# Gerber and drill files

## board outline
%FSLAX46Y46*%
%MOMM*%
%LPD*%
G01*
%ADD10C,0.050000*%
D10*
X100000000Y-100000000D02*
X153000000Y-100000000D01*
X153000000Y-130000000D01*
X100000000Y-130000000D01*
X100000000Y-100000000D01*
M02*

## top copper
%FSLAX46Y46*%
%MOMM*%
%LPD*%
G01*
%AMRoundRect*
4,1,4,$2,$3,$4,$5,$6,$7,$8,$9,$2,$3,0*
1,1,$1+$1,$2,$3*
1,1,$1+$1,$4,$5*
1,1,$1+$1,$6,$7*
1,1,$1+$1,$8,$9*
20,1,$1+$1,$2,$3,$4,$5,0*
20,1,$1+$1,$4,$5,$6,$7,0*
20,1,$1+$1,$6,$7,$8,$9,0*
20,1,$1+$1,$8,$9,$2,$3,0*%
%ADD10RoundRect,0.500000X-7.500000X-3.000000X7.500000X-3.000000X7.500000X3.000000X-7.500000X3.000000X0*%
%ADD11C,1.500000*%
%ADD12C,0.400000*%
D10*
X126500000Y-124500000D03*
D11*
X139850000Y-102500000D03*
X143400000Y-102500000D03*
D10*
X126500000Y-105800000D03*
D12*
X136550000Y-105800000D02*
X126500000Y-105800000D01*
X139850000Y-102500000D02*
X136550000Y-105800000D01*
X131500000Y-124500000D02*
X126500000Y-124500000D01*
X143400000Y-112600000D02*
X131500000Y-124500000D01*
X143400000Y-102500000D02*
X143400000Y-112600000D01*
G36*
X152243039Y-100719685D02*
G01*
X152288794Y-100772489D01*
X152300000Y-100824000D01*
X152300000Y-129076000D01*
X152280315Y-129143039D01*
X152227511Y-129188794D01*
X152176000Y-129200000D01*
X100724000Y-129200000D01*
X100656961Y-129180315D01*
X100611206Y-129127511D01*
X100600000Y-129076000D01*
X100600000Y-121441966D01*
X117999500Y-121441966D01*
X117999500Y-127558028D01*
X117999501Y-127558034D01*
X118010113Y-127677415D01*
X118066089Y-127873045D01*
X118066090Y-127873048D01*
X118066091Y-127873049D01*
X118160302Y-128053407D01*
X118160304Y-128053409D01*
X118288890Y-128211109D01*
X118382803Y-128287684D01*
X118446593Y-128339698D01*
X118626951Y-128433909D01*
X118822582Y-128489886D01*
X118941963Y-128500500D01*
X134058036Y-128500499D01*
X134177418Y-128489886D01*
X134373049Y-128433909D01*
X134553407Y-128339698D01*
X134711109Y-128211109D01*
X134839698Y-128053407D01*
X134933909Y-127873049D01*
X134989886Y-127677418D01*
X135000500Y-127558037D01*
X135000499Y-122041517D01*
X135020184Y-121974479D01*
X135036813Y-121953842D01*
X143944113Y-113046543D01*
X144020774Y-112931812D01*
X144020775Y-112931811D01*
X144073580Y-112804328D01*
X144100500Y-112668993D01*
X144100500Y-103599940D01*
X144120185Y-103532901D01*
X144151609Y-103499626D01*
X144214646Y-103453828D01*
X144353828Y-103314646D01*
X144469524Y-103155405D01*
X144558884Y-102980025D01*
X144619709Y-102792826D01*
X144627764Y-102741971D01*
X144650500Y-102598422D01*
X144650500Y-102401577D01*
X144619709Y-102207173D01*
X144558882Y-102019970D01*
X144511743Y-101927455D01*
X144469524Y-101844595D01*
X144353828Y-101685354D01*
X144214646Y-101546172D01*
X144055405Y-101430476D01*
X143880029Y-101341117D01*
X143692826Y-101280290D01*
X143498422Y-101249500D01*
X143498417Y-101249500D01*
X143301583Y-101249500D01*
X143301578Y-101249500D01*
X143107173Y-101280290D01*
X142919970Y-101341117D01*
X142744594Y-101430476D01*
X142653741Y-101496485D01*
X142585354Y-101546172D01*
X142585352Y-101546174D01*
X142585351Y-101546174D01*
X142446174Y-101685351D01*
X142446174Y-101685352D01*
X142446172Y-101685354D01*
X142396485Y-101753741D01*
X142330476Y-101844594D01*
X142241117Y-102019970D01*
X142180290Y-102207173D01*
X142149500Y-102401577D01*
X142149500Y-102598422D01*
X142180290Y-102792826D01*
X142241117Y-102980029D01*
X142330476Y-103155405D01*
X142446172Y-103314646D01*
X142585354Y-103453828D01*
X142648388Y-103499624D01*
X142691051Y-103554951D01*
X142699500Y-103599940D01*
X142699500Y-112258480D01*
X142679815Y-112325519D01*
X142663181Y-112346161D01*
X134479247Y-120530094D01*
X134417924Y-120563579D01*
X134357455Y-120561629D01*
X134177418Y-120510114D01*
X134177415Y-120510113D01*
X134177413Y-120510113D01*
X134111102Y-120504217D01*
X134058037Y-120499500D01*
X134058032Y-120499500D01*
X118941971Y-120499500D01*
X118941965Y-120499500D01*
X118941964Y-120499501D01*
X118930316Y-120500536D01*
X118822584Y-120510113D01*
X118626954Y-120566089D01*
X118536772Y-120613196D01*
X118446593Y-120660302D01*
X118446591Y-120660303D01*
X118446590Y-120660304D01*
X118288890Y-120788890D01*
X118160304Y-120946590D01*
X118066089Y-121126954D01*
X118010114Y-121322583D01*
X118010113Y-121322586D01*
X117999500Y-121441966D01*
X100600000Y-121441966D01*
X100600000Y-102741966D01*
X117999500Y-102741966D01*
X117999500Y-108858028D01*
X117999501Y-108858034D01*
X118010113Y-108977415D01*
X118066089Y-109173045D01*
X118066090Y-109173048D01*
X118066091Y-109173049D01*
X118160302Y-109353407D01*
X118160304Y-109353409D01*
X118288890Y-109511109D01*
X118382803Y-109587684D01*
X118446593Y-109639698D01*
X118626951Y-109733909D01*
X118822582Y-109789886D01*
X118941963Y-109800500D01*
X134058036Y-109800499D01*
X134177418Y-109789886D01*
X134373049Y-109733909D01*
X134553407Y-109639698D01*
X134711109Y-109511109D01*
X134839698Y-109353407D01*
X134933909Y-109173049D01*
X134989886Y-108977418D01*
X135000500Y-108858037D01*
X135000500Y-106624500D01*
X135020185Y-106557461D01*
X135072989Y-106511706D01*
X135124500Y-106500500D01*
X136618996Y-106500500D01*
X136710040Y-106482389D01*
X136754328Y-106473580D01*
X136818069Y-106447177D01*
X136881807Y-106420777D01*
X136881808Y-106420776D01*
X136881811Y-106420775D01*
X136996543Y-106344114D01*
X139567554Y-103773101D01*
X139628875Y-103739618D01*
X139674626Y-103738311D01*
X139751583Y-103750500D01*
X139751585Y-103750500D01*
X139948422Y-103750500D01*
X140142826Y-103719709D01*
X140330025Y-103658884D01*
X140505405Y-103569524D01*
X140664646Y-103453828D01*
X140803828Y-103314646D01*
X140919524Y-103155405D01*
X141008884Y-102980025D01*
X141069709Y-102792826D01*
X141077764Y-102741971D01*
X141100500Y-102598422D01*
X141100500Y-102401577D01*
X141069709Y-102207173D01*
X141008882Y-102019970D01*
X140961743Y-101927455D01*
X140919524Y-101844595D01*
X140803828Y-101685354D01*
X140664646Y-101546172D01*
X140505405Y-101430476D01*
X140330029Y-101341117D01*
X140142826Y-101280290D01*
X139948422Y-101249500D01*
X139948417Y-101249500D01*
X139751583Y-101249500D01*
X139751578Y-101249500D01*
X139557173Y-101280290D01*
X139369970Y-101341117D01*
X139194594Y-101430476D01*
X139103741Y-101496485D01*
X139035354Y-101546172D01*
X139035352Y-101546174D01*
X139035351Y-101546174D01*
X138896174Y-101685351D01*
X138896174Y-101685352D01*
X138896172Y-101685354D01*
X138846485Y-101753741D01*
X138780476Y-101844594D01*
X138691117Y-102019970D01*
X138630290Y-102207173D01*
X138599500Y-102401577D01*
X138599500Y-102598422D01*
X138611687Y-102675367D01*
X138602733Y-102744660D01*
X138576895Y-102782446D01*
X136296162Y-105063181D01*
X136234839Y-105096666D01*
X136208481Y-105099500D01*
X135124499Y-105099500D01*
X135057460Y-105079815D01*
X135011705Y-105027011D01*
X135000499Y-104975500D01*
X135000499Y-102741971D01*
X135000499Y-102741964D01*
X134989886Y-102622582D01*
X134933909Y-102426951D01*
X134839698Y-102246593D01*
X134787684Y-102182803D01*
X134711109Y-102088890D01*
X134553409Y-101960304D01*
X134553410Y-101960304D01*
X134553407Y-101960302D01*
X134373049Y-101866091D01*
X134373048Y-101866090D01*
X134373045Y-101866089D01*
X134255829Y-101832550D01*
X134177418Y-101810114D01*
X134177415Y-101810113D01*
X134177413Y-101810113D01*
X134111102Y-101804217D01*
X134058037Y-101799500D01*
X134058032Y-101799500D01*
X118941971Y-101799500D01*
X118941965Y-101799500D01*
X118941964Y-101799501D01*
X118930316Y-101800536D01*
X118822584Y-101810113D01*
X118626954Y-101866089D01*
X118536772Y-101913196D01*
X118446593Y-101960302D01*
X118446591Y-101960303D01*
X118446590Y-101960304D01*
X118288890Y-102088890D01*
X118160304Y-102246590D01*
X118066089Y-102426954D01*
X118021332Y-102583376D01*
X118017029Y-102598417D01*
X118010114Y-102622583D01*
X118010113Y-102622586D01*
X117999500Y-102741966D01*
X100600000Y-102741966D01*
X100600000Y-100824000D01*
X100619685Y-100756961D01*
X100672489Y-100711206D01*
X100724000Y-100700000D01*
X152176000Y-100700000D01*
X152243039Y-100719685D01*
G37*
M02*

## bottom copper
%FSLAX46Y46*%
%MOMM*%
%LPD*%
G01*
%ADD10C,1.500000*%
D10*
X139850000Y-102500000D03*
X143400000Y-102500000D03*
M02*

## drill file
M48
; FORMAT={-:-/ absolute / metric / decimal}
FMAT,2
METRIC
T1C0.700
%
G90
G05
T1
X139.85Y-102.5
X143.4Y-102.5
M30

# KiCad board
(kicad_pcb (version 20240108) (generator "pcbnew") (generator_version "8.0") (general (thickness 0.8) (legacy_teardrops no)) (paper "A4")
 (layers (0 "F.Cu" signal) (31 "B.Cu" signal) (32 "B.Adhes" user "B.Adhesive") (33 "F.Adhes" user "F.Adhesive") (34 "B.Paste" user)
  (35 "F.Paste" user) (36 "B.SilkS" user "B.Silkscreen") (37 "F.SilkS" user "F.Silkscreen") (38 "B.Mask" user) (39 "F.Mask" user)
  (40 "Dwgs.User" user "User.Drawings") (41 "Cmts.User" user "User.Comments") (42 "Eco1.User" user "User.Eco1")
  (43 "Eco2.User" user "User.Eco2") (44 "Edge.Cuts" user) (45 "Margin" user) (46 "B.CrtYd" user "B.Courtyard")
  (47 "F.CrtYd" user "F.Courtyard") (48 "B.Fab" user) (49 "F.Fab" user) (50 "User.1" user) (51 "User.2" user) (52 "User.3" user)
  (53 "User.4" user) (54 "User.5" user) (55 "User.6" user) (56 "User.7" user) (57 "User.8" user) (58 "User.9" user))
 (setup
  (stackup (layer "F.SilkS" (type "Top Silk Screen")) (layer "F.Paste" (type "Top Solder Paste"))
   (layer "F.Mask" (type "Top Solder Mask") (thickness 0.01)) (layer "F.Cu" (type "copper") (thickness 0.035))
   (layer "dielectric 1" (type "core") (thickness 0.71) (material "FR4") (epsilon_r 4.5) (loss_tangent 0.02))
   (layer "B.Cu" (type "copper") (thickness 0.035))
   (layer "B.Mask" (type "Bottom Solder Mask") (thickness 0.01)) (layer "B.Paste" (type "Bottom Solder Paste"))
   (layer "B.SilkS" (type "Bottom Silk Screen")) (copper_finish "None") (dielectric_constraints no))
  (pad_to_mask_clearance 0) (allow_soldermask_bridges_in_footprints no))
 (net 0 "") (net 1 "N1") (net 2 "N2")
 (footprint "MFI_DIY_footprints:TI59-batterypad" (layer "F.Cu") (at 126.5 124.5)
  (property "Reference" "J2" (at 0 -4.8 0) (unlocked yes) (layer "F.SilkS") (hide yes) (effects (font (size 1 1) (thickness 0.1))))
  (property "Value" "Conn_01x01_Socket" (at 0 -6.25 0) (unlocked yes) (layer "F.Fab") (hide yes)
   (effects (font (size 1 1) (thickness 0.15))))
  (pad "1" smd roundrect (at 0 0) (size 16 7) (layers "F.Cu" "F.Mask") (roundrect_rratio 0.07142857143) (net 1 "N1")
   (thermal_bridge_angle 45)))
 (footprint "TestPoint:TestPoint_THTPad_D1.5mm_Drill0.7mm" (layer "F.Cu") (at 139.85 102.5 90)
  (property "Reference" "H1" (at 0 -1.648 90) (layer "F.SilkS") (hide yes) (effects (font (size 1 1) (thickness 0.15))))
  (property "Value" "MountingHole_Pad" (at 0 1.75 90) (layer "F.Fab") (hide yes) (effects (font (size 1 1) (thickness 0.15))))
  (pad "1" thru_hole circle (at 0 0 90) (size 1.5 1.5) (drill 0.7) (layers "*.Cu" "*.Mask") (remove_unused_layers no) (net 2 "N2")))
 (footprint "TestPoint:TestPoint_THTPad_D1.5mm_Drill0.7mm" (layer "F.Cu") (at 143.4 102.5 90)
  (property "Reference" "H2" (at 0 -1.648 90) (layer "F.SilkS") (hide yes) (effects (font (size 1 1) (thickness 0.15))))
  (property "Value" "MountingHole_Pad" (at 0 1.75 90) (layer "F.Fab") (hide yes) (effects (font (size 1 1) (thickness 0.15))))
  (pad "1" thru_hole circle (at 0 0 90) (size 1.5 1.5) (drill 0.7) (layers "*.Cu" "*.Mask") (remove_unused_layers no) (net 1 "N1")))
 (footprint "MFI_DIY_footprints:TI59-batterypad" (layer "F.Cu") (at 126.5 105.8)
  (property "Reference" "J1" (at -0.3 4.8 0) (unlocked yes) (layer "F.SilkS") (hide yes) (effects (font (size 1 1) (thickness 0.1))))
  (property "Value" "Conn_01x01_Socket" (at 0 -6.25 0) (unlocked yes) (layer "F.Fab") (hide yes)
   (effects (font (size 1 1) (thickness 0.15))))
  (pad "1" smd roundrect (at 0 0) (size 16 7) (layers "F.Cu" "F.Mask") (roundrect_rratio 0.07142857143) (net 2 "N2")
   (thermal_bridge_angle 45)))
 (gr_rect (start 100 100) (end 153 130) (stroke (width 0.05) (type default)) (fill none) (layer "Edge.Cuts"))
 (segment (start 136.55 105.8) (end 126.5 105.8) (width 0.4) (layer "F.Cu") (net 2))
 (segment (start 139.85 102.5) (end 136.55 105.8) (width 0.4) (layer "F.Cu") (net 2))
 (segment (start 131.5 124.5) (end 126.5 124.5) (width 0.4) (layer "F.Cu") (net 1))
 (segment (start 143.4 112.6) (end 131.5 124.5) (width 0.4) (layer "F.Cu") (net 1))
 (segment (start 143.4 102.5) (end 143.4 112.6) (width 0.4) (layer "F.Cu") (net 1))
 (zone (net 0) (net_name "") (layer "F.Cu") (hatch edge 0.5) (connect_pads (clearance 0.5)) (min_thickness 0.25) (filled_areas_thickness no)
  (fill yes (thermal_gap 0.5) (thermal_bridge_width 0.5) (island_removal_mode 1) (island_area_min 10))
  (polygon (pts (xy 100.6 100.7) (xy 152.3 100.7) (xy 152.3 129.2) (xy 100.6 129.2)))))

